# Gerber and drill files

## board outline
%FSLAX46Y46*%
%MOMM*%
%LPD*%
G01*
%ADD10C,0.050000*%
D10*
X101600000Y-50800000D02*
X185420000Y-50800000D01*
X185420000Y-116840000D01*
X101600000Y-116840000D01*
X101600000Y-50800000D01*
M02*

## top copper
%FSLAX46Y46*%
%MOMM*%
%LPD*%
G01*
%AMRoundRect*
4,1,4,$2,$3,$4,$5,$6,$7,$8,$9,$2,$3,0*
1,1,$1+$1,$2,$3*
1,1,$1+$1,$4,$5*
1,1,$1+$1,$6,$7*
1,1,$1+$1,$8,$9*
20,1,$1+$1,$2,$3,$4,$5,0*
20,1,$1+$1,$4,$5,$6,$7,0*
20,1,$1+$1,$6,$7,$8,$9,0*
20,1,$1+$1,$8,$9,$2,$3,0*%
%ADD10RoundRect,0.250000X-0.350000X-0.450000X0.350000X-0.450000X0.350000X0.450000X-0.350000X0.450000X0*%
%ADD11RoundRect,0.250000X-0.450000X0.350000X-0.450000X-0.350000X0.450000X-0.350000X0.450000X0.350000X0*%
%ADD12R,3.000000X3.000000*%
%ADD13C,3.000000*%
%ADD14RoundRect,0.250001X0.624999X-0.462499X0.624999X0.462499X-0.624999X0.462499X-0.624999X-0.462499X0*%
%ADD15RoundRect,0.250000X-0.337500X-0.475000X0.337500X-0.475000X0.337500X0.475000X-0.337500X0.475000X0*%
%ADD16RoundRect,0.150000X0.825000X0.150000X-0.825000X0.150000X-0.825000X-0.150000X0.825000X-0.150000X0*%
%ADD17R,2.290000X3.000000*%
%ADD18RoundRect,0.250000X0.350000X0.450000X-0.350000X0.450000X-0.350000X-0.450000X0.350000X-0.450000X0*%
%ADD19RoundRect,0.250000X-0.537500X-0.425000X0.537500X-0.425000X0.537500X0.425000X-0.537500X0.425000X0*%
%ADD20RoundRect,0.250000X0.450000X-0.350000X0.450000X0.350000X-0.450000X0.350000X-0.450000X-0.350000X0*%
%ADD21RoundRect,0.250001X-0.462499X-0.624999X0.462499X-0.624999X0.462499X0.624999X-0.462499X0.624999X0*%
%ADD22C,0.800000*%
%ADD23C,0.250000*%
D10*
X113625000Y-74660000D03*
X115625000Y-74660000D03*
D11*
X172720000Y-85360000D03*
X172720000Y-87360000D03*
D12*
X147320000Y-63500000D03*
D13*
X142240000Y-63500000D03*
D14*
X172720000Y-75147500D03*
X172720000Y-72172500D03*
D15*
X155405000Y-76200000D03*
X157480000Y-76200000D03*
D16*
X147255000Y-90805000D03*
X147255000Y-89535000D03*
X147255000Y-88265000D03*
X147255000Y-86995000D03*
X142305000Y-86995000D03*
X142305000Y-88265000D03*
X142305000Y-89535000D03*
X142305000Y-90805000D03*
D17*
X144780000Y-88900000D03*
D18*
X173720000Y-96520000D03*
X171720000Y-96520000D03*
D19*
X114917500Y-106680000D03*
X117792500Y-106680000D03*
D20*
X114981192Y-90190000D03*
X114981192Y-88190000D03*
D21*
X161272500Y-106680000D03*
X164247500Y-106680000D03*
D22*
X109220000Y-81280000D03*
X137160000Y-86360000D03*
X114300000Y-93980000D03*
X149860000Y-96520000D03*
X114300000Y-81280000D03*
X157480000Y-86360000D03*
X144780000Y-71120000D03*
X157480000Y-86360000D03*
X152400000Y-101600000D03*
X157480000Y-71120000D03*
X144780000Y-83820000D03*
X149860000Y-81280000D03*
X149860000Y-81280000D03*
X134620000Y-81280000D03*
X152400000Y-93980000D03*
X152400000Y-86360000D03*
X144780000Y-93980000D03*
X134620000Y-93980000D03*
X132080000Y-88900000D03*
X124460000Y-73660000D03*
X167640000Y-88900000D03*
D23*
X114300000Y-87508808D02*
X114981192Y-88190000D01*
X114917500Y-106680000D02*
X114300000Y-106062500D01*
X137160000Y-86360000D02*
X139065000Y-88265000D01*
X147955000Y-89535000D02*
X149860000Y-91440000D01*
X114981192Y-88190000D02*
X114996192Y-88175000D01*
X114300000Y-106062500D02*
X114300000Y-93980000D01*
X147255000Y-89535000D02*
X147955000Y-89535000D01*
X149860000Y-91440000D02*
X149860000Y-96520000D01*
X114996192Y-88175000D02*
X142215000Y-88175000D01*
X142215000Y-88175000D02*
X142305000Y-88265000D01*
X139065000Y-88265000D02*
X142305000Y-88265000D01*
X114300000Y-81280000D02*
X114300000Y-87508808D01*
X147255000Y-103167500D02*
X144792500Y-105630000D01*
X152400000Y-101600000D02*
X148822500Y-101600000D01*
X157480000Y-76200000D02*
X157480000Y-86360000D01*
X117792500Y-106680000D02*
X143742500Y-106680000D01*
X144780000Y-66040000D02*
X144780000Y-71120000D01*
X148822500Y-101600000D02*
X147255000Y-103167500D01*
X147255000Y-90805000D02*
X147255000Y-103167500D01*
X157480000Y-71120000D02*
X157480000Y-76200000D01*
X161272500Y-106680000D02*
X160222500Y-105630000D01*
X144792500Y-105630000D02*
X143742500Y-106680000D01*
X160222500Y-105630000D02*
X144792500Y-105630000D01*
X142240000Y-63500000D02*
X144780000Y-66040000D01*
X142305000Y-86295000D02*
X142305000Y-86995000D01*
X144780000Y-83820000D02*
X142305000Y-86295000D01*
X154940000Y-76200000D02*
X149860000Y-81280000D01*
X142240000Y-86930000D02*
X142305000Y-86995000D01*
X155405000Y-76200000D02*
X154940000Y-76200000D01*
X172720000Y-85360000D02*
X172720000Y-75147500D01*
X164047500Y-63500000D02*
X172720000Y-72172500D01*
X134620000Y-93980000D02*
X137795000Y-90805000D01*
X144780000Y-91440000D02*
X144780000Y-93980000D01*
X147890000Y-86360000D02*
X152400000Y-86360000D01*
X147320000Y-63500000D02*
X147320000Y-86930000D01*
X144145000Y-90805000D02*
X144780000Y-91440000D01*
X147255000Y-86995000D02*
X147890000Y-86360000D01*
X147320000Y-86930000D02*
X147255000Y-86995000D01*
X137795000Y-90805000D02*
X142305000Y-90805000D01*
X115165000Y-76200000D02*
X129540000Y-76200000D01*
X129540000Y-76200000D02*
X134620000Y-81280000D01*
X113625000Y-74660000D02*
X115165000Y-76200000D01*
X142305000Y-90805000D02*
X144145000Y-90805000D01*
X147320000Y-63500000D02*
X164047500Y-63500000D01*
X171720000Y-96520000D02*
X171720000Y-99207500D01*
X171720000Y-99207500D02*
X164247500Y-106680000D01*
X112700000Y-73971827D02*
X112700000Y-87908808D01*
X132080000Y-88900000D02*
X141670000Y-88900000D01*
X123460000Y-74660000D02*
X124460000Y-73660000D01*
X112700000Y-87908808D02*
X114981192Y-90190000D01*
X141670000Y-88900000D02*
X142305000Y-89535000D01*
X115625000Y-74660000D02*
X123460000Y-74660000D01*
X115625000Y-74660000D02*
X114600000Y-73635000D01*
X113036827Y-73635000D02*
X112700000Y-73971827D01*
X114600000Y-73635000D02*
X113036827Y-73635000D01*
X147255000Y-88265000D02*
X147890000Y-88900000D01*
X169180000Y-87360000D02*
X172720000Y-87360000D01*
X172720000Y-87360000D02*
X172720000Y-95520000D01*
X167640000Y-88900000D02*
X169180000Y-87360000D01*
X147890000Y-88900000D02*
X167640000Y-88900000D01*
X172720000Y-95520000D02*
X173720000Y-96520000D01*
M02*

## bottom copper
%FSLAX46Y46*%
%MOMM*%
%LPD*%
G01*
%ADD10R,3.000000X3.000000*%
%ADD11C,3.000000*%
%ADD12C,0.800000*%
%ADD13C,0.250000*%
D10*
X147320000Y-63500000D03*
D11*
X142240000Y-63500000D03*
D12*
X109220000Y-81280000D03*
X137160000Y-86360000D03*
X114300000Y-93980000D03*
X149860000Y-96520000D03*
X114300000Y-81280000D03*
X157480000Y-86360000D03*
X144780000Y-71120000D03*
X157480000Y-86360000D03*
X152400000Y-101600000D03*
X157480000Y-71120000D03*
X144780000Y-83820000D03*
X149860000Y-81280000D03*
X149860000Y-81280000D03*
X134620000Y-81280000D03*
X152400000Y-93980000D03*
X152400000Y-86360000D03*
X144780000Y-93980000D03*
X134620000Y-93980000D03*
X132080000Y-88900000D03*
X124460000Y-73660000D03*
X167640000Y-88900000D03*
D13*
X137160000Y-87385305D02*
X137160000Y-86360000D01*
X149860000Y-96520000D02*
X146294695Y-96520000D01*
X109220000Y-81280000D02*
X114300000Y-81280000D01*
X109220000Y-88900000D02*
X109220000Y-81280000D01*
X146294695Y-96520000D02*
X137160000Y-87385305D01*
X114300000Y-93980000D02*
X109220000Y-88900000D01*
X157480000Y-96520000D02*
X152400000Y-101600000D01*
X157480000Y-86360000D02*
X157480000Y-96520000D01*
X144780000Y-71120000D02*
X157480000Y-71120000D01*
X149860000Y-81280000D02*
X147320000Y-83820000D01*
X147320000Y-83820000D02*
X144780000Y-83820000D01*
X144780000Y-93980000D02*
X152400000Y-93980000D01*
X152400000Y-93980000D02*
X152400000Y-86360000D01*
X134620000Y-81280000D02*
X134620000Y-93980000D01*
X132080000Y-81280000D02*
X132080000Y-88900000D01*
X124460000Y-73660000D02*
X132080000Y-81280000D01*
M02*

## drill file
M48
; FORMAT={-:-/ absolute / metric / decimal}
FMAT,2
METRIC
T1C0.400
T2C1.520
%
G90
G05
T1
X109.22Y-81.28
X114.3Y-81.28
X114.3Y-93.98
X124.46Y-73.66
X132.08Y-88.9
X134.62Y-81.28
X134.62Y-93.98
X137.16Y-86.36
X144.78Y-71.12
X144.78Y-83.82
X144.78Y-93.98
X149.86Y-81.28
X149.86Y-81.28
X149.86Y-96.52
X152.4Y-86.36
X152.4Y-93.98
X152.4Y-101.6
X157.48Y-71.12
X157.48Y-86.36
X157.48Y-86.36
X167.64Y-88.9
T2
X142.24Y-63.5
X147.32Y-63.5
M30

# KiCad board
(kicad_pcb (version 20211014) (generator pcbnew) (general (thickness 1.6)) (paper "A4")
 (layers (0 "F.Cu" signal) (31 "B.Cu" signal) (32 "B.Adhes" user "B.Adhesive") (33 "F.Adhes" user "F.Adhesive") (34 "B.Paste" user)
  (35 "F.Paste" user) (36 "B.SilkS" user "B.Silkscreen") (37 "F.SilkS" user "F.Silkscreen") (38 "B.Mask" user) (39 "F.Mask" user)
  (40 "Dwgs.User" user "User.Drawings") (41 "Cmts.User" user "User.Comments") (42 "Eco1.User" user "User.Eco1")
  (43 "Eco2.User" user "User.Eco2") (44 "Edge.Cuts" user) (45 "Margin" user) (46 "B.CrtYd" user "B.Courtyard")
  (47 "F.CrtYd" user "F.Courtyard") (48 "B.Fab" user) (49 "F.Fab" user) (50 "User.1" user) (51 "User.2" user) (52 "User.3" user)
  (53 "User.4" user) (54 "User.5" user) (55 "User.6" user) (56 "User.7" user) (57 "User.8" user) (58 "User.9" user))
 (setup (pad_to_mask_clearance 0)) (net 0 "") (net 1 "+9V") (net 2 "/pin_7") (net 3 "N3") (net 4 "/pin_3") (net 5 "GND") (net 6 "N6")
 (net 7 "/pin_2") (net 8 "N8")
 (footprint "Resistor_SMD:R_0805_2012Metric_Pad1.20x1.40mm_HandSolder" (layer "F.Cu") (at 114.625 74.66)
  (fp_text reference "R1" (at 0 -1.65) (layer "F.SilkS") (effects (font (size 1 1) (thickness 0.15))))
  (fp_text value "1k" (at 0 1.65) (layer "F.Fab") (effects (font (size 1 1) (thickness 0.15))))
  (pad "1" smd roundrect (at -1 0) (size 1.2 1.4) (layers "F.Cu" "F.Paste" "F.Mask") (roundrect_rratio 0.208333) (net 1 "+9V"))
  (pad "2" smd roundrect (at 1 0) (size 1.2 1.4) (layers "F.Cu" "F.Paste" "F.Mask") (roundrect_rratio 0.208333) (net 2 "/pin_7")))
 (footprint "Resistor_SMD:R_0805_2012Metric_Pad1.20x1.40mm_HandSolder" (layer "F.Cu") (at 172.72 86.36 -90)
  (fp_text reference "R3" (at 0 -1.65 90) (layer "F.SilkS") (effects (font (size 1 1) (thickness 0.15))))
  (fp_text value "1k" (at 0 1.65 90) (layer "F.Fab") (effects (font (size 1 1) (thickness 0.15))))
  (pad "1" smd roundrect (at -1 0 270) (size 1.2 1.4) (layers "F.Cu" "F.Paste" "F.Mask") (roundrect_rratio 0.208333) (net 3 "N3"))
  (pad "2" smd roundrect (at 1 0 270) (size 1.2 1.4) (layers "F.Cu" "F.Paste" "F.Mask") (roundrect_rratio 0.208333) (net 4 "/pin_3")))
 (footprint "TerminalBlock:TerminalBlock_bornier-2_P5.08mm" (layer "F.Cu") (at 147.32 63.5 180)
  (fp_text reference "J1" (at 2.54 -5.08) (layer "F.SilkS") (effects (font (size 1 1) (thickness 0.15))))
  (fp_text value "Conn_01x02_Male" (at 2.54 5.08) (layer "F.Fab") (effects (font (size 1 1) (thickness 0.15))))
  (pad "1" thru_hole rect (at 0 0 180) (size 3 3) (drill 1.52) (layers *.Cu *.Mask) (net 1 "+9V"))
  (pad "2" thru_hole circle (at 5.08 0 180) (size 3 3) (drill 1.52) (layers *.Cu *.Mask) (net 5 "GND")))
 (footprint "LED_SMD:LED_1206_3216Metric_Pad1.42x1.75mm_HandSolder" (layer "F.Cu") (at 172.72 73.66 90)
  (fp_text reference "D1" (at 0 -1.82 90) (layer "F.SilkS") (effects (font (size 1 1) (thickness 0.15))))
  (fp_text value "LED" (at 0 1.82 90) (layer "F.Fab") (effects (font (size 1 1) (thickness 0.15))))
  (pad "1" smd roundrect (at -1.4875 0 90) (size 1.425 1.75) (layers "F.Cu" "F.Paste" "F.Mask") (roundrect_rratio 0.175439) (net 3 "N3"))
  (pad "2" smd roundrect (at 1.4875 0 90) (size 1.425 1.75) (layers "F.Cu" "F.Paste" "F.Mask") (roundrect_rratio 0.175439) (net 1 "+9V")))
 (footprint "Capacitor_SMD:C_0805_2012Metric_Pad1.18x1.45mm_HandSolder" (layer "F.Cu") (at 156.4425 76.2)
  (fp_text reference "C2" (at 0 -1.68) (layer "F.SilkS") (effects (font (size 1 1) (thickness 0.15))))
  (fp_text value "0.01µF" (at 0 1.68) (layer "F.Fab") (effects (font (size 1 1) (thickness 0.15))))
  (pad "1" smd roundrect (at -1.0375 0) (size 1.175 1.45) (layers "F.Cu" "F.Paste" "F.Mask") (roundrect_rratio 0.212766) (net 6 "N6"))
  (pad "2" smd roundrect (at 1.0375 0) (size 1.175 1.45) (layers "F.Cu" "F.Paste" "F.Mask") (roundrect_rratio 0.212766) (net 5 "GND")))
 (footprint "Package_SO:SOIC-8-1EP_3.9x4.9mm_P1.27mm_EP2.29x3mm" (layer "F.Cu") (at 144.78 88.9 180)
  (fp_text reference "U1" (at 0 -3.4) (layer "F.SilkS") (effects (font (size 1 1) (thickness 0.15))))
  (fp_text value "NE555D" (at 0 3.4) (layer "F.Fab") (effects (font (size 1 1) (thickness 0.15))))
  (pad "" smd roundrect (at 0.57 -0.75 180) (size 0.92 1.21) (layers "F.Paste") (roundrect_rratio 0.25))
  (pad "" smd roundrect (at 0.57 0.75 180) (size 0.92 1.21) (layers "F.Paste") (roundrect_rratio 0.25))
  (pad "" smd roundrect (at -0.57 -0.75 180) (size 0.92 1.21) (layers "F.Paste" "B.SilkS") (roundrect_rratio 0.25))
  (pad "" smd roundrect (at -0.57 0.75 180) (size 0.92 1.21) (layers "F.Paste") (roundrect_rratio 0.25))
  (pad "1" smd roundrect (at -2.475 -1.905 180) (size 1.95 0.6) (layers "F.Cu" "F.Paste" "F.Mask") (roundrect_rratio 0.25) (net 5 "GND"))
  (pad "2" smd roundrect (at -2.475 -0.635 180) (size 1.95 0.6) (layers "F.Cu" "F.Paste" "F.Mask") (roundrect_rratio 0.25) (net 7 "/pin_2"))
  (pad "3" smd roundrect (at -2.475 0.635 180) (size 1.95 0.6) (layers "F.Cu" "F.Paste" "F.Mask") (roundrect_rratio 0.25) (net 4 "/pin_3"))
  (pad "4" smd roundrect (at -2.475 1.905 180) (size 1.95 0.6) (layers "F.Cu" "F.Paste" "F.Mask") (roundrect_rratio 0.25) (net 1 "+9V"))
  (pad "5" smd roundrect (at 2.475 1.905 180) (size 1.95 0.6) (layers "F.Cu" "F.Paste" "F.Mask") (roundrect_rratio 0.25) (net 6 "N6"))
  (pad "6" smd roundrect (at 2.475 0.635 180) (size 1.95 0.6) (layers "F.Cu" "F.Paste" "F.Mask") (roundrect_rratio 0.25) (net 7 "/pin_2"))
  (pad "7" smd roundrect (at 2.475 -0.635 180) (size 1.95 0.6) (layers "F.Cu" "F.Paste" "F.Mask") (roundrect_rratio 0.25) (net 2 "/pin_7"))
  (pad "8" smd roundrect (at 2.475 -1.905 180) (size 1.95 0.6) (layers "F.Cu" "F.Paste" "F.Mask") (roundrect_rratio 0.25) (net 1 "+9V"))
  (pad "9" smd rect (at 0 0 180) (size 2.29 3) (layers "F.Cu" "F.Mask")))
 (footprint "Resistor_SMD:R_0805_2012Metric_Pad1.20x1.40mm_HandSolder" (layer "F.Cu") (at 172.72 96.52 180)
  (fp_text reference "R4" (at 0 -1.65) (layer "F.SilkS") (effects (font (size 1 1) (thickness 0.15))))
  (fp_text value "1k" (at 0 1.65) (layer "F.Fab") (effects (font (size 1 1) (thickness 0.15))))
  (pad "1" smd roundrect (at -1 0 180) (size 1.2 1.4) (layers "F.Cu" "F.Paste" "F.Mask") (roundrect_rratio 0.208333) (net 4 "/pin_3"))
  (pad "2" smd roundrect (at 1 0 180) (size 1.2 1.4) (layers "F.Cu" "F.Paste" "F.Mask") (roundrect_rratio 0.208333) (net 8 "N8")))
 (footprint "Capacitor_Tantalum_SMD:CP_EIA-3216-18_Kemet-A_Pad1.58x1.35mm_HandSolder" (layer "F.Cu") (at 116.355 106.68)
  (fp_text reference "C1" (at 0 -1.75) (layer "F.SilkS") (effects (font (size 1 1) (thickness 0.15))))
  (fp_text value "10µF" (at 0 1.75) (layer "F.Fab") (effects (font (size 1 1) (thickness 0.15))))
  (pad "1" smd roundrect (at -1.4375 0) (size 1.575 1.35) (layers "F.Cu" "F.Paste" "F.Mask") (roundrect_rratio 0.185185) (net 7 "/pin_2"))
  (pad "2" smd roundrect (at 1.4375 0) (size 1.575 1.35) (layers "F.Cu" "F.Paste" "F.Mask") (roundrect_rratio 0.185185) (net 5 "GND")))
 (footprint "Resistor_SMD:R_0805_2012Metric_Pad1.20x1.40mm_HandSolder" (layer "F.Cu") (at 114.981192 89.19 90)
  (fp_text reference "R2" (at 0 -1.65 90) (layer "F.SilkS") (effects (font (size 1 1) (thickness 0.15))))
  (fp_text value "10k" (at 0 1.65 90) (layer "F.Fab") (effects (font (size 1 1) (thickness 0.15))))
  (pad "1" smd roundrect (at -1 0 90) (size 1.2 1.4) (layers "F.Cu" "F.Paste" "F.Mask") (roundrect_rratio 0.208333) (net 2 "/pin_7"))
  (pad "2" smd roundrect (at 1 0 90) (size 1.2 1.4) (layers "F.Cu" "F.Paste" "F.Mask") (roundrect_rratio 0.208333) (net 7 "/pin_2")))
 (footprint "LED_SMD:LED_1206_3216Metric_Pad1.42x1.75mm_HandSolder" (layer "F.Cu") (at 162.76 106.68)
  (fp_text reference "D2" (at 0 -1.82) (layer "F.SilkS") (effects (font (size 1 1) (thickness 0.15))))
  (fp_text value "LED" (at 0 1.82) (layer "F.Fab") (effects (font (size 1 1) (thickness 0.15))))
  (pad "1" smd roundrect (at -1.4875 0) (size 1.425 1.75) (layers "F.Cu" "F.Paste" "F.Mask") (roundrect_rratio 0.175439) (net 5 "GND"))
  (pad "2" smd roundrect (at 1.4875 0) (size 1.425 1.75) (layers "F.Cu" "F.Paste" "F.Mask") (roundrect_rratio 0.175439) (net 8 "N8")))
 (gr_rect (start 101.6 50.8) (end 185.42 116.84) (layer "Edge.Cuts") (width 0.05) (fill none))
 (segment (start 114.3 87.508808) (end 114.981192 88.19) (width 0.25) (layer "F.Cu") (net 7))
 (segment (start 114.9175 106.68) (end 114.3 106.0625) (width 0.25) (layer "F.Cu") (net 7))
 (segment (start 137.16 86.36) (end 139.065 88.265) (width 0.25) (layer "F.Cu") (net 7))
 (segment (start 147.955 89.535) (end 149.86 91.44) (width 0.25) (layer "F.Cu") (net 7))
 (segment (start 114.981192 88.19) (end 114.996192 88.175) (width 0.25) (layer "F.Cu") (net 7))
 (segment (start 114.3 106.0625) (end 114.3 93.98) (width 0.25) (layer "F.Cu") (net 7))
 (segment (start 147.255 89.535) (end 147.955 89.535) (width 0.25) (layer "F.Cu") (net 7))
 (segment (start 149.86 91.44) (end 149.86 96.52) (width 0.25) (layer "F.Cu") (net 7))
 (segment (start 114.996192 88.175) (end 142.215 88.175) (width 0.25) (layer "F.Cu") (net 7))
 (segment (start 142.215 88.175) (end 142.305 88.265) (width 0.25) (layer "F.Cu") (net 7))
 (segment (start 139.065 88.265) (end 142.305 88.265) (width 0.25) (layer "F.Cu") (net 7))
 (segment (start 114.3 81.28) (end 114.3 87.508808) (width 0.25) (layer "F.Cu") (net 7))
 (via (at 109.22 81.28) (size 0.8) (drill 0.4) (layers "F.Cu" "B.Cu") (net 7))
 (via (at 137.16 86.36) (size 0.8) (drill 0.4) (layers "F.Cu" "B.Cu") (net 7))
 (via (at 114.3 93.98) (size 0.8) (drill 0.4) (layers "F.Cu" "B.Cu") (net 7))
 (via (at 149.86 96.52) (size 0.8) (drill 0.4) (layers "F.Cu" "B.Cu") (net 7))
 (via (at 114.3 81.28) (size 0.8) (drill 0.4) (layers "F.Cu" "B.Cu") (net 7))
 (segment (start 137.16 87.385305) (end 137.16 86.36) (width 0.25) (layer "B.Cu") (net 7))
 (segment (start 149.86 96.52) (end 146.294695 96.52) (width 0.25) (layer "B.Cu") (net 7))
 (segment (start 109.22 81.28) (end 114.3 81.28) (width 0.25) (layer "B.Cu") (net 7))
 (segment (start 109.22 88.9) (end 109.22 81.28) (width 0.25) (layer "B.Cu") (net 7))
 (segment (start 146.294695 96.52) (end 137.16 87.385305) (width 0.25) (layer "B.Cu") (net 7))
 (segment (start 114.3 93.98) (end 109.22 88.9) (width 0.25) (layer "B.Cu") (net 7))
 (segment (start 147.255 103.1675) (end 144.7925 105.63) (width 0.25) (layer "F.Cu") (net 5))
 (segment (start 152.4 101.6) (end 148.8225 101.6) (width 0.25) (layer "F.Cu") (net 5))
 (segment (start 157.48 76.2) (end 157.48 86.36) (width 0.25) (layer "F.Cu") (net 5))
 (segment (start 117.7925 106.68) (end 143.7425 106.68) (width 0.25) (layer "F.Cu") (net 5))
 (segment (start 144.78 66.04) (end 144.78 71.12) (width 0.25) (layer "F.Cu") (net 5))
 (segment (start 148.8225 101.6) (end 147.255 103.1675) (width 0.25) (layer "F.Cu") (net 5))
 (segment (start 147.255 90.805) (end 147.255 103.1675) (width 0.25) (layer "F.Cu") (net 5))
 (segment (start 157.48 71.12) (end 157.48 76.2) (width 0.25) (layer "F.Cu") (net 5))
 (segment (start 161.2725 106.68) (end 160.2225 105.63) (width 0.25) (layer "F.Cu") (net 5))
 (segment (start 144.7925 105.63) (end 143.7425 106.68) (width 0.25) (layer "F.Cu") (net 5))
 (segment (start 160.2225 105.63) (end 144.7925 105.63) (width 0.25) (layer "F.Cu") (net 5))
 (segment (start 142.24 63.5) (end 144.78 66.04) (width 0.25) (layer "F.Cu") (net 5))
 (via (at 157.48 86.36) (size 0.8) (drill 0.4) (layers "F.Cu" "B.Cu") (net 5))
 (via (at 144.78 71.12) (size 0.8) (drill 0.4) (layers "F.Cu" "B.Cu") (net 5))
 (via (at 157.48 86.36) (size 0.8) (drill 0.4) (layers "F.Cu" "B.Cu") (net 5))
 (via (at 152.4 101.6) (size 0.8) (drill 0.4) (layers "F.Cu" "B.Cu") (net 5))
 (via (at 157.48 71.12) (size 0.8) (drill 0.4) (layers "F.Cu" "B.Cu") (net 5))
 (segment (start 157.48 96.52) (end 152.4 101.6) (width 0.25) (layer "B.Cu") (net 5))
 (segment (start 157.48 86.36) (end 157.48 96.52) (width 0.25) (layer "B.Cu") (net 5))
 (segment (start 144.78 71.12) (end 157.48 71.12) (width 0.25) (layer "B.Cu") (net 5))
 (segment (start 142.305 86.295) (end 142.305 86.995) (width 0.25) (layer "F.Cu") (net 6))
 (segment (start 144.78 83.82) (end 142.305 86.295) (width 0.25) (layer "F.Cu") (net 6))
 (segment (start 154.94 76.2) (end 149.86 81.28) (width 0.25) (layer "F.Cu") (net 6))
 (segment (start 142.24 86.93) (end 142.305 86.995) (width 0.25) (layer "F.Cu") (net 6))
 (segment (start 155.405 76.2) (end 154.94 76.2) (width 0.25) (layer "F.Cu") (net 6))
 (via (at 144.78 83.82) (size 0.8) (drill 0.4) (layers "F.Cu" "B.Cu") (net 6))
 (via (at 149.86 81.28) (size 0.8) (drill 0.4) (layers "F.Cu" "B.Cu") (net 6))
 (via (at 149.86 81.28) (size 0.8) (drill 0.4) (layers "F.Cu" "B.Cu") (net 6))
 (segment (start 149.86 81.28) (end 147.32 83.82) (width 0.25) (layer "B.Cu") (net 6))
 (segment (start 147.32 83.82) (end 144.78 83.82) (width 0.25) (layer "B.Cu") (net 6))
 (segment (start 172.72 85.36) (end 172.72 75.1475) (width 0.25) (layer "F.Cu") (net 3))
 (segment (start 164.0475 63.5) (end 172.72 72.1725) (width 0.25) (layer "F.Cu") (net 1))
 (segment (start 134.62 93.98) (end 137.795 90.805) (width 0.25) (layer "F.Cu") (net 1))
 (segment (start 144.78 91.44) (end 144.78 93.98) (width 0.25) (layer "F.Cu") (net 1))
 (segment (start 147.89 86.36) (end 152.4 86.36) (width 0.25) (layer "F.Cu") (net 1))
 (segment (start 147.32 63.5) (end 147.32 86.93) (width 0.25) (layer "F.Cu") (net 1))
 (segment (start 144.145 90.805) (end 144.78 91.44) (width 0.25) (layer "F.Cu") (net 1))
 (segment (start 147.255 86.995) (end 147.89 86.36) (width 0.25) (layer "F.Cu") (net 1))
 (segment (start 147.32 86.93) (end 147.255 86.995) (width 0.25) (layer "F.Cu") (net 1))
 (segment (start 137.795 90.805) (end 142.305 90.805) (width 0.25) (layer "F.Cu") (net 1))
 (segment (start 115.165 76.2) (end 129.54 76.2) (width 0.25) (layer "F.Cu") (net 1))
 (segment (start 129.54 76.2) (end 134.62 81.28) (width 0.25) (layer "F.Cu") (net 1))
 (segment (start 113.625 74.66) (end 115.165 76.2) (width 0.25) (layer "F.Cu") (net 1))
 (segment (start 142.305 90.805) (end 144.145 90.805) (width 0.25) (layer "F.Cu") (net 1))
 (segment (start 147.32 63.5) (end 164.0475 63.5) (width 0.25) (layer "F.Cu") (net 1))
 (via (at 134.62 81.28) (size 0.8) (drill 0.4) (layers "F.Cu" "B.Cu") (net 1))
 (via (at 152.4 93.98) (size 0.8) (drill 0.4) (layers "F.Cu" "B.Cu") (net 1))
 (via (at 152.4 86.36) (size 0.8) (drill 0.4) (layers "F.Cu" "B.Cu") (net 1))
 (via (at 144.78 93.98) (size 0.8) (drill 0.4) (layers "F.Cu" "B.Cu") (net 1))
 (via (at 134.62 93.98) (size 0.8) (drill 0.4) (layers "F.Cu" "B.Cu") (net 1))
 (segment (start 144.78 93.98) (end 152.4 93.98) (width 0.25) (layer "B.Cu") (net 1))
 (segment (start 152.4 93.98) (end 152.4 86.36) (width 0.25) (layer "B.Cu") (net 1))
 (segment (start 134.62 81.28) (end 134.62 93.98) (width 0.25) (layer "B.Cu") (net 1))
 (segment (start 171.72 96.52) (end 171.72 99.2075) (width 0.25) (layer "F.Cu") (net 8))
 (segment (start 171.72 99.2075) (end 164.2475 106.68) (width 0.25) (layer "F.Cu") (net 8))
 (segment (start 112.7 73.971827) (end 112.7 87.908808) (width 0.25) (layer "F.Cu") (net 2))
 (segment (start 132.08 88.9) (end 141.67 88.9) (width 0.25) (layer "F.Cu") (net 2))
 (segment (start 123.46 74.66) (end 124.46 73.66) (width 0.25) (layer "F.Cu") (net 2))
 (segment (start 112.7 87.908808) (end 114.981192 90.19) (width 0.25) (layer "F.Cu") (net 2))
 (segment (start 141.67 88.9) (end 142.305 89.535) (width 0.25) (layer "F.Cu") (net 2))
 (segment (start 115.625 74.66) (end 123.46 74.66) (width 0.25) (layer "F.Cu") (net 2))
 (segment (start 115.625 74.66) (end 114.6 73.635) (width 0.25) (layer "F.Cu") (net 2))
 (segment (start 113.036827 73.635) (end 112.7 73.971827) (width 0.25) (layer "F.Cu") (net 2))
 (segment (start 114.6 73.635) (end 113.036827 73.635) (width 0.25) (layer "F.Cu") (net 2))
 (via (at 132.08 88.9) (size 0.8) (drill 0.4) (layers "F.Cu" "B.Cu") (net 2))
 (via (at 124.46 73.66) (size 0.8) (drill 0.4) (layers "F.Cu" "B.Cu") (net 2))
 (segment (start 132.08 81.28) (end 132.08 88.9) (width 0.25) (layer "B.Cu") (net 2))
 (segment (start 124.46 73.66) (end 132.08 81.28) (width 0.25) (layer "B.Cu") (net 2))
 (segment (start 147.255 88.265) (end 147.89 88.9) (width 0.25) (layer "F.Cu") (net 4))
 (segment (start 169.18 87.36) (end 172.72 87.36) (width 0.25) (layer "F.Cu") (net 4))
 (segment (start 172.72 87.36) (end 172.72 95.52) (width 0.25) (layer "F.Cu") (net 4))
 (segment (start 167.64 88.9) (end 169.18 87.36) (width 0.25) (layer "F.Cu") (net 4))
 (segment (start 147.89 88.9) (end 167.64 88.9) (width 0.25) (layer "F.Cu") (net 4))
 (segment (start 172.72 95.52) (end 173.72 96.52) (width 0.25) (layer "F.Cu") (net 4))
 (via (at 167.64 88.9) (size 0.8) (drill 0.4) (layers "F.Cu" "B.Cu") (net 4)))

